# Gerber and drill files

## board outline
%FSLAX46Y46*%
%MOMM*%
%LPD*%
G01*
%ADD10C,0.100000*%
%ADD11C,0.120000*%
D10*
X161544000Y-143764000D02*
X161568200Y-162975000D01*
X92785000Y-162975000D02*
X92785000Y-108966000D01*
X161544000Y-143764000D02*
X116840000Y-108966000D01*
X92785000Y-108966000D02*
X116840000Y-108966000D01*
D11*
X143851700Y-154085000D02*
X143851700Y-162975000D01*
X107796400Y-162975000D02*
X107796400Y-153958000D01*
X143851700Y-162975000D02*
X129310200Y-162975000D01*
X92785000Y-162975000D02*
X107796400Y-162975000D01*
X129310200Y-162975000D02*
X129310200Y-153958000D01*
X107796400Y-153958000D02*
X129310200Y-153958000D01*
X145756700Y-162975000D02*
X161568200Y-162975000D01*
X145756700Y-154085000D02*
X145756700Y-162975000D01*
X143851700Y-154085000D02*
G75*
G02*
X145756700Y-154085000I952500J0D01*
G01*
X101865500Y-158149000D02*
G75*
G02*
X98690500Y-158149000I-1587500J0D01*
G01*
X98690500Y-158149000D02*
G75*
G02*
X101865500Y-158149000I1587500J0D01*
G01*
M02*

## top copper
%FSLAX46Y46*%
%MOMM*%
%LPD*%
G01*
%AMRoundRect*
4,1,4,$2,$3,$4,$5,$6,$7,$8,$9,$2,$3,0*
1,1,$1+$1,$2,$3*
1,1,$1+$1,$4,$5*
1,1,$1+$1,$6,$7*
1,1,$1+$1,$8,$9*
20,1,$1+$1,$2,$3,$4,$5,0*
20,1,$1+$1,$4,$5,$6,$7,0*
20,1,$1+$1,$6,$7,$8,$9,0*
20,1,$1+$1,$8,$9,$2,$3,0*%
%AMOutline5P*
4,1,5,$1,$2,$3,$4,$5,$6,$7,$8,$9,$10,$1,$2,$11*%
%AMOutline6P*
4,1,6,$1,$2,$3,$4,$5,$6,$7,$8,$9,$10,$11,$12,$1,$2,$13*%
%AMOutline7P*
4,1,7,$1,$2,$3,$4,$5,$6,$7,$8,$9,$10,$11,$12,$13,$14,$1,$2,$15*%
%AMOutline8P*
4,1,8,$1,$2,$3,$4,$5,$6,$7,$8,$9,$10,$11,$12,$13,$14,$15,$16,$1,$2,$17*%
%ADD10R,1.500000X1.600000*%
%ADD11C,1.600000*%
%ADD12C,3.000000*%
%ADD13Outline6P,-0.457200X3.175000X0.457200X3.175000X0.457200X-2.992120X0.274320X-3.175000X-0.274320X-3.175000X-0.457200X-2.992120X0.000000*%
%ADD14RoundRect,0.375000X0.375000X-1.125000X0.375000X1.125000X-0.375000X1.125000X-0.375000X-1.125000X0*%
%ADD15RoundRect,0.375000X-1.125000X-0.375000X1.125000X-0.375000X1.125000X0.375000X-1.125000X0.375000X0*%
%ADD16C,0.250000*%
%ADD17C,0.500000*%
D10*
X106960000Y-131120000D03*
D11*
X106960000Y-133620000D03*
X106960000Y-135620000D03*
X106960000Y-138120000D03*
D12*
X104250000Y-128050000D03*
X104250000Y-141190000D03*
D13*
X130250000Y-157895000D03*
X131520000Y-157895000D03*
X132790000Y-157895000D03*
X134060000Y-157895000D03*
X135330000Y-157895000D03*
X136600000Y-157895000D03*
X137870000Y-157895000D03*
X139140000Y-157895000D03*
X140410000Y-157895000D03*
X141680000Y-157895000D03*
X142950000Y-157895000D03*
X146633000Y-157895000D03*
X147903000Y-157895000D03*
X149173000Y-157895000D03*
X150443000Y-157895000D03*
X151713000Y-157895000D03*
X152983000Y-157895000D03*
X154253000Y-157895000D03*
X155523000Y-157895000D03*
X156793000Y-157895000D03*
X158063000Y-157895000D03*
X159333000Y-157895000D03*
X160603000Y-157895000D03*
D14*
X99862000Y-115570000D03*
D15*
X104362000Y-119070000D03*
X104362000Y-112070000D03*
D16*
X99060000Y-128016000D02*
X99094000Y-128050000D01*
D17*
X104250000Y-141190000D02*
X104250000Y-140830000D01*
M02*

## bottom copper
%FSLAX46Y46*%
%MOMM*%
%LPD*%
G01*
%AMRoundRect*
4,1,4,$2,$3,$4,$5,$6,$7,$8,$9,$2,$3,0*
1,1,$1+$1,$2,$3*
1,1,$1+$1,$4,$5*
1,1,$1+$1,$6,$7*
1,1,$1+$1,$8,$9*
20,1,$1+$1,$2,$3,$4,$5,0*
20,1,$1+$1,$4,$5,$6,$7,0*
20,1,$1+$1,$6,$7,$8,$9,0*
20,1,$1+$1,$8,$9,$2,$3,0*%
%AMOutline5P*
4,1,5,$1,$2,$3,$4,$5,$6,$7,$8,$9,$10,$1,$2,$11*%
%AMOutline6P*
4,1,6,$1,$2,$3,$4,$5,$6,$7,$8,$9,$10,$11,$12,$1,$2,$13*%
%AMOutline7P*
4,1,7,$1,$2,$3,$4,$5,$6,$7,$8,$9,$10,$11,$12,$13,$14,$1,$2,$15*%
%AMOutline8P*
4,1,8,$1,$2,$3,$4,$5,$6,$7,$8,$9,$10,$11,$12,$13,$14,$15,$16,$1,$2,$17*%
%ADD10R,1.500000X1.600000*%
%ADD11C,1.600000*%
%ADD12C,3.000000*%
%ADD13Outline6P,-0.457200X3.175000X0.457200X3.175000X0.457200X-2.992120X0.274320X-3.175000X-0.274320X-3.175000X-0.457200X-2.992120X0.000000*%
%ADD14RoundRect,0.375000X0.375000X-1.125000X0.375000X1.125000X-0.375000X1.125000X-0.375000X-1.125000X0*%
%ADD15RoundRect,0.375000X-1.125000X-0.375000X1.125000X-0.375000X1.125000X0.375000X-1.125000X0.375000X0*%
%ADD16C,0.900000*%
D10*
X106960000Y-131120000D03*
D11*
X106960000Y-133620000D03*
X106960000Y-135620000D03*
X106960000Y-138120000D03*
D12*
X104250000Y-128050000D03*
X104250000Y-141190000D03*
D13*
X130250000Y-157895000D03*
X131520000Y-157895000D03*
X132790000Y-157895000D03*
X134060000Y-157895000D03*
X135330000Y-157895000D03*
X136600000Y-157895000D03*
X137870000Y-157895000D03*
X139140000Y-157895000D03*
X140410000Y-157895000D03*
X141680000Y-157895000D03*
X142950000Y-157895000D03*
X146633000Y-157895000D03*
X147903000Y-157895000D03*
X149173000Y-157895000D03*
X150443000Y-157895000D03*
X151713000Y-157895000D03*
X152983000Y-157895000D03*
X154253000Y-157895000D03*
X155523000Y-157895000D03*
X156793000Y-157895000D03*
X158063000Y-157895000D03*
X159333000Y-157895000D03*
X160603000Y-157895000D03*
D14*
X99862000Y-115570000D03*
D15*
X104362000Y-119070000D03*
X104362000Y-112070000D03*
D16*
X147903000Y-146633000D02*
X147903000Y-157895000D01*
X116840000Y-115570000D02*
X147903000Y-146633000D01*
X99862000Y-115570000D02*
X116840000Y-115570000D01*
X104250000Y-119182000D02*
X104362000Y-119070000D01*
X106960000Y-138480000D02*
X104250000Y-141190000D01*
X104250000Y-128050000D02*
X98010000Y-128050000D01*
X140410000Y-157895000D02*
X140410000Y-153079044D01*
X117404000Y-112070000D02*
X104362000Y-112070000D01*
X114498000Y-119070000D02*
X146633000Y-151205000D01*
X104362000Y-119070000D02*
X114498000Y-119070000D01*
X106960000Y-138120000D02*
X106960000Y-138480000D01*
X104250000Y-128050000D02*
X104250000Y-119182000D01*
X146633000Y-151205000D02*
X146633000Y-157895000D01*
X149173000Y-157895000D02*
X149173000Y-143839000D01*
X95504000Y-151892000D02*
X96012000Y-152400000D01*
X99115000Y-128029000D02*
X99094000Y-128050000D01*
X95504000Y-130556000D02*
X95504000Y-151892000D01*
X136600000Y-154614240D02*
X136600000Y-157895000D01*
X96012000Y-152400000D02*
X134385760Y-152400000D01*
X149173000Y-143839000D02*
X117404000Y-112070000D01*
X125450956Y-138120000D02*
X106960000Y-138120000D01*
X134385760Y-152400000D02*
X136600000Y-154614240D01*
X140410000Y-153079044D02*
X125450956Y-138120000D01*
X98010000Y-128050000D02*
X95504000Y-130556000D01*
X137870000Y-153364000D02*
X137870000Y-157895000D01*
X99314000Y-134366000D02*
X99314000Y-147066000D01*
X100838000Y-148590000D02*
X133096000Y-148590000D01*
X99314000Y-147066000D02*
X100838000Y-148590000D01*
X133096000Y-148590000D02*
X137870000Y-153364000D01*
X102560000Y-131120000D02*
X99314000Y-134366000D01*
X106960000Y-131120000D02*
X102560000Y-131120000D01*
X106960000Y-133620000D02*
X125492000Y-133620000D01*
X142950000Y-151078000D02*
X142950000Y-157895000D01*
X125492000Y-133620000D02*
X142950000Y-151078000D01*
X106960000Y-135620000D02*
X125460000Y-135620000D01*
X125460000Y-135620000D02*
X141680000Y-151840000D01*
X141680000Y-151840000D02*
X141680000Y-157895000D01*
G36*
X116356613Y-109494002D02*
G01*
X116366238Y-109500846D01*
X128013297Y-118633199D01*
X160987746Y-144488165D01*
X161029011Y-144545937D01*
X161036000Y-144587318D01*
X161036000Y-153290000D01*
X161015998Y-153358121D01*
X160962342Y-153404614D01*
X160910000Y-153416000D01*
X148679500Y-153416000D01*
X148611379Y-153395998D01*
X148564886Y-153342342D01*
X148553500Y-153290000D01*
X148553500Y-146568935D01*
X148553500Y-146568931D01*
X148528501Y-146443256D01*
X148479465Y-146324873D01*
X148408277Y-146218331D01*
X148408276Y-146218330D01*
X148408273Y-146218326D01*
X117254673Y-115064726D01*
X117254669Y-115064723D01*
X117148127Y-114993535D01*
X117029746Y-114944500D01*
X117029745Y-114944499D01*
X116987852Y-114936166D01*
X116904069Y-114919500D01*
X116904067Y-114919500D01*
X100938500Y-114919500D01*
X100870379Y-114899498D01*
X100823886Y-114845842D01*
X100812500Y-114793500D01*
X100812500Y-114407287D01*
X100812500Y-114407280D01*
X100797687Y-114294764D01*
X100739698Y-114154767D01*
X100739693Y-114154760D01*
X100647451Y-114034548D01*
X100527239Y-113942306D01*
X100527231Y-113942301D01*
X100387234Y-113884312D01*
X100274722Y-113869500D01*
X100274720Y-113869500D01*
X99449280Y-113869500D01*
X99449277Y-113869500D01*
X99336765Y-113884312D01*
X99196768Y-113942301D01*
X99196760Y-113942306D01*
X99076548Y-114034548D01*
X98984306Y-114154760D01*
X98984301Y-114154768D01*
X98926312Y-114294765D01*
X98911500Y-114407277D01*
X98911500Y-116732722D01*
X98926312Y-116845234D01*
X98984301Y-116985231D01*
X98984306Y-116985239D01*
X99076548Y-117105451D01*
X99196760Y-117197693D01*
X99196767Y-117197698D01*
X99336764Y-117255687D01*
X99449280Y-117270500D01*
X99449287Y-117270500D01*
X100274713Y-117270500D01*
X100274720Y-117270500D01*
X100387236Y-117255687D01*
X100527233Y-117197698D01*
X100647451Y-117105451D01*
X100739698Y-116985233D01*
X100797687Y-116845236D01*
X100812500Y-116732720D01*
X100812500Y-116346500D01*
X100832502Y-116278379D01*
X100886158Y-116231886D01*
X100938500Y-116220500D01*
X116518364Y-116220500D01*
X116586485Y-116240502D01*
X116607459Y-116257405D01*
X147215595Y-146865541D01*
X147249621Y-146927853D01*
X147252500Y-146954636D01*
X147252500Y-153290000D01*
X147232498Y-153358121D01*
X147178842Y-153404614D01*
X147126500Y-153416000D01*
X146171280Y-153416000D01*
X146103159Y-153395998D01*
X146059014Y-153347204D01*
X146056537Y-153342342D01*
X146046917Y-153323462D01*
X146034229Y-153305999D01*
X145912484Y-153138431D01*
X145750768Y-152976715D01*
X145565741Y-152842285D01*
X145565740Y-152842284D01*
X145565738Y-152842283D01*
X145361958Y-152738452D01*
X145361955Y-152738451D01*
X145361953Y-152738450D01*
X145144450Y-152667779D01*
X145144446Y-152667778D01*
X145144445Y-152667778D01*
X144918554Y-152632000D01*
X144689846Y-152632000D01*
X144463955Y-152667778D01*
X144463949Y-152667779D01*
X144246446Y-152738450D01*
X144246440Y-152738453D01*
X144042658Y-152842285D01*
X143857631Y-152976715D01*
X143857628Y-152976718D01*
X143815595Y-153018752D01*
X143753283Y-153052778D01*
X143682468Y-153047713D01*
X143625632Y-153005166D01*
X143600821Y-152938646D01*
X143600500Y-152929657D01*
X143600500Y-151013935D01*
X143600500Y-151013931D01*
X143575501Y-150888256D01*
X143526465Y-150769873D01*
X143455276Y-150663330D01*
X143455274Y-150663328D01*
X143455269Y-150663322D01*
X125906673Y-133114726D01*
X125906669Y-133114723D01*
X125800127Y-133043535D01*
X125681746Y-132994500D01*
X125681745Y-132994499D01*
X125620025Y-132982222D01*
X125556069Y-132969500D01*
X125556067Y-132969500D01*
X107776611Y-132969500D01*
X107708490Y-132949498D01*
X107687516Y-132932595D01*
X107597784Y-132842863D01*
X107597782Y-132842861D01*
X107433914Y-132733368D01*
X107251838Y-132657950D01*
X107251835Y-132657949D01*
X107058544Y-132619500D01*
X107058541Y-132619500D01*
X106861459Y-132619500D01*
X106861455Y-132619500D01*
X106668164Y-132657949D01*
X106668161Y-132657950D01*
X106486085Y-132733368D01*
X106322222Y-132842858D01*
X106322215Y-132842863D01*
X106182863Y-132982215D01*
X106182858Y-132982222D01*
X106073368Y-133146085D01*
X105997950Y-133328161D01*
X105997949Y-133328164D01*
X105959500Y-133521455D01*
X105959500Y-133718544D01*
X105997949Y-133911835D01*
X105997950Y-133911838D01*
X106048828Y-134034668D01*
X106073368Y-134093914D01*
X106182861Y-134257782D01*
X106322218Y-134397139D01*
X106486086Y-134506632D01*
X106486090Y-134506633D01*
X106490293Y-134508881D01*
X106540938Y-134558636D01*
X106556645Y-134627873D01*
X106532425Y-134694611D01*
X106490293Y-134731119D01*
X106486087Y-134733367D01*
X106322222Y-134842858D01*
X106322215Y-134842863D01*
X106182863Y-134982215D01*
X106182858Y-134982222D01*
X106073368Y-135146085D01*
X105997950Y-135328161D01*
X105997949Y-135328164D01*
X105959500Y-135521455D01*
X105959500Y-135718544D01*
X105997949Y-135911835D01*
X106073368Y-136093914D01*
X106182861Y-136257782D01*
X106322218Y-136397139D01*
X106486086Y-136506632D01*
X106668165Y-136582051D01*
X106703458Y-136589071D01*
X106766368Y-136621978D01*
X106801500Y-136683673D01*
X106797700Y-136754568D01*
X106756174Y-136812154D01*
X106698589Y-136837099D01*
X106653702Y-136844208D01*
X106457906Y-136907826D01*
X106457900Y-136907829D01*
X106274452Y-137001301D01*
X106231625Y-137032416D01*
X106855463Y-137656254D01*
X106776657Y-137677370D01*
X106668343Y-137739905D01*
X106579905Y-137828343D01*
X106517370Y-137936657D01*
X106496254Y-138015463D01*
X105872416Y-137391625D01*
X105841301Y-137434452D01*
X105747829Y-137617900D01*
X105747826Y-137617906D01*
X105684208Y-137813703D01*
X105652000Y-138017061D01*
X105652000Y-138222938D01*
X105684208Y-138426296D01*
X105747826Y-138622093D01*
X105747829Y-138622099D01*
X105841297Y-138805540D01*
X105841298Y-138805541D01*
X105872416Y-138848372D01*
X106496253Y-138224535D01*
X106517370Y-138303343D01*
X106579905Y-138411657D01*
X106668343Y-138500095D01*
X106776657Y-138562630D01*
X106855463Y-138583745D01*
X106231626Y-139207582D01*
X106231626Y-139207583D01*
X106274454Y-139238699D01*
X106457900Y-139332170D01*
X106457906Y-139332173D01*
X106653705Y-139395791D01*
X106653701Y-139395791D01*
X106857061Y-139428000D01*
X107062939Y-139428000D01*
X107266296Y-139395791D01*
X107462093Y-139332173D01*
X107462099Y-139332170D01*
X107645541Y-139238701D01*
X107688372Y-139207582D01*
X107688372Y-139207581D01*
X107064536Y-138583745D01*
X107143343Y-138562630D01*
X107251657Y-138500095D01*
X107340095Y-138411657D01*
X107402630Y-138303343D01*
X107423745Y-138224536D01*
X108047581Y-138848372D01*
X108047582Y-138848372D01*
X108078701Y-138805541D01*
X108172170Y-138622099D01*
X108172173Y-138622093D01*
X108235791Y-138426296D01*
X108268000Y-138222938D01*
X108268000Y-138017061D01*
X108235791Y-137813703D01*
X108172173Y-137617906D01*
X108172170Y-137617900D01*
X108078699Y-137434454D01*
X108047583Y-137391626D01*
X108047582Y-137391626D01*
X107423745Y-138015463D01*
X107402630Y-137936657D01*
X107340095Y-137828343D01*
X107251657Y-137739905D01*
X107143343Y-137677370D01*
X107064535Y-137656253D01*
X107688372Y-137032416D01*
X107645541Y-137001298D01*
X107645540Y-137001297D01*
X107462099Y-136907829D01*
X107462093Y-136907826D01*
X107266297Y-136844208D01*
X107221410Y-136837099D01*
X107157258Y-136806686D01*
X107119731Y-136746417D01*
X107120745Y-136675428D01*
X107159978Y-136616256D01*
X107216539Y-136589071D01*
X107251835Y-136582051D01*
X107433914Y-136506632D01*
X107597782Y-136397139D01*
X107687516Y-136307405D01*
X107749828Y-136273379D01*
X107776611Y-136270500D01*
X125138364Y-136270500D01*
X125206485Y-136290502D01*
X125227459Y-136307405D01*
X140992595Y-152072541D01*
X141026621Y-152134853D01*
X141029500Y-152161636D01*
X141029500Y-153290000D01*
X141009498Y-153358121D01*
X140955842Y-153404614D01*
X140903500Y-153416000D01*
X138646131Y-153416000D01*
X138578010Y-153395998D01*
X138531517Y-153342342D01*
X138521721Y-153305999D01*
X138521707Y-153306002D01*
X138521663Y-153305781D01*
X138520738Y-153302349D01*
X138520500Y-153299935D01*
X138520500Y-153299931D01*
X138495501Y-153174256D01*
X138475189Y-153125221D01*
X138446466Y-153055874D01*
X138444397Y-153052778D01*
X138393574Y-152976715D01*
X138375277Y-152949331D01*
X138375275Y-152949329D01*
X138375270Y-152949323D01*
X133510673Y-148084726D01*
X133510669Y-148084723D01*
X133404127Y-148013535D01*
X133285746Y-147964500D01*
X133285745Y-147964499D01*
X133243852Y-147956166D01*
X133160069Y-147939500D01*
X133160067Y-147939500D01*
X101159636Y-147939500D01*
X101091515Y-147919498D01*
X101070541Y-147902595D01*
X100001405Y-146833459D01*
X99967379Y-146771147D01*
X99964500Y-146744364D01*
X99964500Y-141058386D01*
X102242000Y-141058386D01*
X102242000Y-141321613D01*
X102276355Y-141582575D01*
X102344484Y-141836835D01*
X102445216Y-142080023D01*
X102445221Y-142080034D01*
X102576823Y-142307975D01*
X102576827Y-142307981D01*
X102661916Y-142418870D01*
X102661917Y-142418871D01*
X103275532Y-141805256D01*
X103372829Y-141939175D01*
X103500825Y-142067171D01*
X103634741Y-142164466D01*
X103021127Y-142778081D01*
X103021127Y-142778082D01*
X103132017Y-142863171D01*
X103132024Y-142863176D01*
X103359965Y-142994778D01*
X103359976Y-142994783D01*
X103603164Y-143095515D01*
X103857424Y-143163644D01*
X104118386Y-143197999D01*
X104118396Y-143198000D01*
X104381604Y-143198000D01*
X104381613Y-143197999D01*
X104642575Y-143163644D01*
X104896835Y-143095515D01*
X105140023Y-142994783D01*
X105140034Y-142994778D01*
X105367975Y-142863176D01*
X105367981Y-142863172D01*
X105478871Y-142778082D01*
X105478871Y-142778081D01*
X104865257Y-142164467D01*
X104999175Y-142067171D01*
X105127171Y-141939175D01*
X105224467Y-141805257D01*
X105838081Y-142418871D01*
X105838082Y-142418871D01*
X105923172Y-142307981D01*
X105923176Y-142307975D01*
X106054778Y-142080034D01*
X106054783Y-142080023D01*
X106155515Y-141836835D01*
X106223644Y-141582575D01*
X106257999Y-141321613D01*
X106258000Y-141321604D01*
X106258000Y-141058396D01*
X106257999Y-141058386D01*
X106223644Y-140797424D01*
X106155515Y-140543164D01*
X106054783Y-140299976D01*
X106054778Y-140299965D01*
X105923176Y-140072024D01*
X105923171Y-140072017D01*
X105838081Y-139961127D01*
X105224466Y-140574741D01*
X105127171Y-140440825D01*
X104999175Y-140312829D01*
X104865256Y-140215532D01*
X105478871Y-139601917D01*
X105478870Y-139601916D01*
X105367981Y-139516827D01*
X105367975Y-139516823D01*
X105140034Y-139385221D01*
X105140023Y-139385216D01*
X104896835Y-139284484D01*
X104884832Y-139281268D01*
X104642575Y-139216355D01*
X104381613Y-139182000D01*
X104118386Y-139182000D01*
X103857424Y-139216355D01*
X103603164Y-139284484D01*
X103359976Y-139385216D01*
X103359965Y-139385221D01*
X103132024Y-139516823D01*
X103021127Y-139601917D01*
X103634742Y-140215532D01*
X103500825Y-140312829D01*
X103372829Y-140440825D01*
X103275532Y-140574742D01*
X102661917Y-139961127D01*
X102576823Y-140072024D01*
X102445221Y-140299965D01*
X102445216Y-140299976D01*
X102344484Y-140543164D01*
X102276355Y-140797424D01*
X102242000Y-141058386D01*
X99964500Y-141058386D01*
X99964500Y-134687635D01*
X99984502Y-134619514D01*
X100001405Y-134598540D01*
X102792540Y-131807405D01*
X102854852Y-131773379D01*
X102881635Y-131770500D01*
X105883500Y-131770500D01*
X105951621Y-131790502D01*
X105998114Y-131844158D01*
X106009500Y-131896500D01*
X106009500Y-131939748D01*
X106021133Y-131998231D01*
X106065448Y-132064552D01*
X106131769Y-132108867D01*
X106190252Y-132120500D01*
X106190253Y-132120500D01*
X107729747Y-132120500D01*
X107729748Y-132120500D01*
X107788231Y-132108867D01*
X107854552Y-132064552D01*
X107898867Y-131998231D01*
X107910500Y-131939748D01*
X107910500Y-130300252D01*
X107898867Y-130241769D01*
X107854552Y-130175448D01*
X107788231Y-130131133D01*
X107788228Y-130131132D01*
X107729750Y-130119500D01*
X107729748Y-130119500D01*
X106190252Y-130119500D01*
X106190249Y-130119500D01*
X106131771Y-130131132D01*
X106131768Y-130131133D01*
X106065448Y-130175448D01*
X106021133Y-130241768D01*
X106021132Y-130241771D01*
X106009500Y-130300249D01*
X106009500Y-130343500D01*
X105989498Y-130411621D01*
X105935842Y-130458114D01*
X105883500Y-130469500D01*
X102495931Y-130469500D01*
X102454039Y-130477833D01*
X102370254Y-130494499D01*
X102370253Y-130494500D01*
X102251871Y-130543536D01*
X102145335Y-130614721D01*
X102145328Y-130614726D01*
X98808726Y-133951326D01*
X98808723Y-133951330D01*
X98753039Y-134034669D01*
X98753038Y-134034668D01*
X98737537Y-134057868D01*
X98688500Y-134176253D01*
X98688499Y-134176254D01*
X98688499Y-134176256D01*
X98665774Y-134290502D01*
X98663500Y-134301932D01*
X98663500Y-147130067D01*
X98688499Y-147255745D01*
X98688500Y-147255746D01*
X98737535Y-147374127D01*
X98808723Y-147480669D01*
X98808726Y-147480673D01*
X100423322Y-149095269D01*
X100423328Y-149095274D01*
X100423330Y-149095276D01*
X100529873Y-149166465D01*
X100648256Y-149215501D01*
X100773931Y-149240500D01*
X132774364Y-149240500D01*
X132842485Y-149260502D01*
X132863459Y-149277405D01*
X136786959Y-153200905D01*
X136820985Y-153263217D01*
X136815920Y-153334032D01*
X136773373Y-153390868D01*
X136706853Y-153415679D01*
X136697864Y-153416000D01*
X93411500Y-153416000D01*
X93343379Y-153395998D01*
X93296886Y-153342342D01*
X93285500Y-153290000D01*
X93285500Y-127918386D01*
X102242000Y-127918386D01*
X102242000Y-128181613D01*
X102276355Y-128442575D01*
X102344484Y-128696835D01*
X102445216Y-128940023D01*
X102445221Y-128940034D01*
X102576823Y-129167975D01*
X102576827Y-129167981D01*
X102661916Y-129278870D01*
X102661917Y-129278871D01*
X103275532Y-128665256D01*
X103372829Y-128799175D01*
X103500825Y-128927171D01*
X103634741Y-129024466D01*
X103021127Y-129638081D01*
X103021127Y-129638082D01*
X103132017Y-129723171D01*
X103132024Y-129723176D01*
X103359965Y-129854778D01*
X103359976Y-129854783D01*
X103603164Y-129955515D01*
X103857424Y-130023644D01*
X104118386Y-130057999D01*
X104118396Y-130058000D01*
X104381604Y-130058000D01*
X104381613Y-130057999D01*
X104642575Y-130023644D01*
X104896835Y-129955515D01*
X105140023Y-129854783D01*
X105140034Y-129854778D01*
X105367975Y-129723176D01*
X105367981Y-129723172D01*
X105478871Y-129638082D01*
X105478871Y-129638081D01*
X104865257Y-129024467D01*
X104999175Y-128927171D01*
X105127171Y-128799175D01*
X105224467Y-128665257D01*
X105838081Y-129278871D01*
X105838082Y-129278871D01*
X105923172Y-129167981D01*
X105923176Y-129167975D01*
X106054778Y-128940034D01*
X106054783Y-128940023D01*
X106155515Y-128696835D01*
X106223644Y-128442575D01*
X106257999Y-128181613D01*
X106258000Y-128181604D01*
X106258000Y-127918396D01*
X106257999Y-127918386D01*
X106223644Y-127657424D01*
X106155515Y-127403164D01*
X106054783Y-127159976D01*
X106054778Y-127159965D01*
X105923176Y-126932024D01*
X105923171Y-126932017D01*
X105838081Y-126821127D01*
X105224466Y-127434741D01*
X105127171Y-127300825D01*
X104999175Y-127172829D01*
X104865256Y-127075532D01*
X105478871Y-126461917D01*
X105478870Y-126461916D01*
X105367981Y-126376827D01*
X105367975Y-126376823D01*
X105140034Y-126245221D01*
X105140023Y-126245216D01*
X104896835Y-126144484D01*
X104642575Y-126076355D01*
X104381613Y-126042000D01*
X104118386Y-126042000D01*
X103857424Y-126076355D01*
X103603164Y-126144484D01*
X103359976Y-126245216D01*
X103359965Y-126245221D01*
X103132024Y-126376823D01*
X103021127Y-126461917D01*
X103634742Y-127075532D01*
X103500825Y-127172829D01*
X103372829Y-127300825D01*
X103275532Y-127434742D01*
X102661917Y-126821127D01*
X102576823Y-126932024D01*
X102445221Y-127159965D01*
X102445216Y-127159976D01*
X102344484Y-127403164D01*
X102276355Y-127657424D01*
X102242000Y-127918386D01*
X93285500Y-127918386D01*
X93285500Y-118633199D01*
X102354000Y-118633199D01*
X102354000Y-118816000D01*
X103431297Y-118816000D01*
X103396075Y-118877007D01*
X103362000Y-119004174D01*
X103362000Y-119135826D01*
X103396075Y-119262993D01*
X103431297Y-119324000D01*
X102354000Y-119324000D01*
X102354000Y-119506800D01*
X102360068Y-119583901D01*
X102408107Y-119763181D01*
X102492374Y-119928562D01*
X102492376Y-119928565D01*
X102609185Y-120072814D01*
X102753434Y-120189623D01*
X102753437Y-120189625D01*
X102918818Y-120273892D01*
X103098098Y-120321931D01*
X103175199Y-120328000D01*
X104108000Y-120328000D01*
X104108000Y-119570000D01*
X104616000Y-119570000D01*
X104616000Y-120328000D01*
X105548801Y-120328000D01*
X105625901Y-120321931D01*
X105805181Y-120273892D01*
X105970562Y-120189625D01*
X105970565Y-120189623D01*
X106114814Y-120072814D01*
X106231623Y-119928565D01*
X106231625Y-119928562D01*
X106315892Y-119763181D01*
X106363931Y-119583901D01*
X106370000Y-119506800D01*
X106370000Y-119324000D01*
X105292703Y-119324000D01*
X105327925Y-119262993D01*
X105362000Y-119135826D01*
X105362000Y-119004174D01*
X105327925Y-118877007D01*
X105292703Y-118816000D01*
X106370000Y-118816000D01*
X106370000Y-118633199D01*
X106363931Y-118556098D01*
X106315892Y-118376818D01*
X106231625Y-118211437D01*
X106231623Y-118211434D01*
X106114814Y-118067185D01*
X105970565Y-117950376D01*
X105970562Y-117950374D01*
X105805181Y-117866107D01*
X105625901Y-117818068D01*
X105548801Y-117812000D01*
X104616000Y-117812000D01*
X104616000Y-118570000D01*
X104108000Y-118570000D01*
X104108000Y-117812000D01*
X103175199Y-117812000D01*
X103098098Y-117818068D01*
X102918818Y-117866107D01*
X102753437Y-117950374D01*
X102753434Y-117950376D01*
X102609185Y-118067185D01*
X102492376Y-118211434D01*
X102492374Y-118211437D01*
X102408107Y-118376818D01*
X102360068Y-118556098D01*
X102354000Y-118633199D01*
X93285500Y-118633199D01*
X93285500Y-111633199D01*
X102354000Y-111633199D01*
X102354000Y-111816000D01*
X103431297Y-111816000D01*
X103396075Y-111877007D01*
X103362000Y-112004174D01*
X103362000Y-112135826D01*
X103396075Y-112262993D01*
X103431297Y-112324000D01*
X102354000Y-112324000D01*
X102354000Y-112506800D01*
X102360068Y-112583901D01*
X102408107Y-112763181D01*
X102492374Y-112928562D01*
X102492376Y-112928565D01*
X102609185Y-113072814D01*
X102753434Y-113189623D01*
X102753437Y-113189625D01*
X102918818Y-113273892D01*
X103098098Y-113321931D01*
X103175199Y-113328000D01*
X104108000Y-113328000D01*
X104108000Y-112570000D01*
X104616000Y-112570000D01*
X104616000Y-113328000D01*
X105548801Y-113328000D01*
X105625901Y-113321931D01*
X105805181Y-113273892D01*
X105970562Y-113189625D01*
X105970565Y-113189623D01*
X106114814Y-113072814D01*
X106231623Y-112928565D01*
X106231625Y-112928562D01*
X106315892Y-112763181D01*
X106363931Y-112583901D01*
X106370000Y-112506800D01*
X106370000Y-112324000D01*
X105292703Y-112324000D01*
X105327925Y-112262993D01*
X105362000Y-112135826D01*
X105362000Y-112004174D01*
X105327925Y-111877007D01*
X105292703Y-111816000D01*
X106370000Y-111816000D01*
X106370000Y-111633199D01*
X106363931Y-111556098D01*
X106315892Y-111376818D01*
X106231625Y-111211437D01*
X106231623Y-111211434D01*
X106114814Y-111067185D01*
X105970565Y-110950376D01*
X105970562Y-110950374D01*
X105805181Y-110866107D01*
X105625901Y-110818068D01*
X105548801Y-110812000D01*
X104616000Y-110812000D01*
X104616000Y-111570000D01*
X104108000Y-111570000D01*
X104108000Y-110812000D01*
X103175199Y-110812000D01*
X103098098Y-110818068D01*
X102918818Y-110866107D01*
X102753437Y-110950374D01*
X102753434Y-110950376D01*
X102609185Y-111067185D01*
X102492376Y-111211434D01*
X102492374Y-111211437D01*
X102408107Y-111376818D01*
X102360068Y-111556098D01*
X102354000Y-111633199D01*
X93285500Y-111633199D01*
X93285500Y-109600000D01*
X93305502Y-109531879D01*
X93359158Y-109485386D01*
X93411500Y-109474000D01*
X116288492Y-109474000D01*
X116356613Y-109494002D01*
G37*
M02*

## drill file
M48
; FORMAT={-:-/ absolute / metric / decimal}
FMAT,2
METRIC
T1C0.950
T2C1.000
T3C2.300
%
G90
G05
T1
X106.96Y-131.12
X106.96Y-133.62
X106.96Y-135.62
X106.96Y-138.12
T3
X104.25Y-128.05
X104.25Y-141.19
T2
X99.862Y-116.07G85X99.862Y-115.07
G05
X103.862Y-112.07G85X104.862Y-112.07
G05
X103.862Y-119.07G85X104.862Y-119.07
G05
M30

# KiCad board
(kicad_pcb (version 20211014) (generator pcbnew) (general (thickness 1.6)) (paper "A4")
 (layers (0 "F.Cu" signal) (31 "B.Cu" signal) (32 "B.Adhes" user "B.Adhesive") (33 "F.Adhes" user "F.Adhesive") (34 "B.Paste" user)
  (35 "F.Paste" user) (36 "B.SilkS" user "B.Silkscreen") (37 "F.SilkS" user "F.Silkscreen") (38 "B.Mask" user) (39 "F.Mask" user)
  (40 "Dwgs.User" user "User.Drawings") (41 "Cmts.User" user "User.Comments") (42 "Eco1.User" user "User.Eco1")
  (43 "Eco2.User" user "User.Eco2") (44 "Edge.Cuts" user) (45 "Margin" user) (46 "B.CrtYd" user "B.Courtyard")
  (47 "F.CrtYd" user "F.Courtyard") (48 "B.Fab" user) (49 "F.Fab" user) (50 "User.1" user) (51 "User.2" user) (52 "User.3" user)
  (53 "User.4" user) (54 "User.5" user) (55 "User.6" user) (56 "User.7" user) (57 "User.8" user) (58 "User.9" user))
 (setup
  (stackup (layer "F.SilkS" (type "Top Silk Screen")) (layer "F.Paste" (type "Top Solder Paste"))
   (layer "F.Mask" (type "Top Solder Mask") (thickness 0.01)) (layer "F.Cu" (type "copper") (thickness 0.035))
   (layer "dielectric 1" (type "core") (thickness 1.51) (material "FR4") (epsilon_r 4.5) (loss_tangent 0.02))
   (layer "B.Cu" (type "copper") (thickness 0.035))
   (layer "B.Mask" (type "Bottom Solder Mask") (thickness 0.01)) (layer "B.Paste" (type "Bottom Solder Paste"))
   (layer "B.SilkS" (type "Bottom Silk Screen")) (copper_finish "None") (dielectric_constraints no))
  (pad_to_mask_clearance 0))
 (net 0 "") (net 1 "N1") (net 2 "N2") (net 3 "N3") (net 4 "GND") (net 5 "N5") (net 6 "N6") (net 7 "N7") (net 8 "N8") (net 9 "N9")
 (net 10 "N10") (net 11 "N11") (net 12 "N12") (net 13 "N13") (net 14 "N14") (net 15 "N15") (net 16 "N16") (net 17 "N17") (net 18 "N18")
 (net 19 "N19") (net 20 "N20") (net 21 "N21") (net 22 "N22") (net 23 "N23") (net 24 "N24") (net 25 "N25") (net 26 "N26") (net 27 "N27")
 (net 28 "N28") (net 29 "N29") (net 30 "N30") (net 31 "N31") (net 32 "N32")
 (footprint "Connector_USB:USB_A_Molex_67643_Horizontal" (layer "F.Cu") (at 106.96 131.12 -90)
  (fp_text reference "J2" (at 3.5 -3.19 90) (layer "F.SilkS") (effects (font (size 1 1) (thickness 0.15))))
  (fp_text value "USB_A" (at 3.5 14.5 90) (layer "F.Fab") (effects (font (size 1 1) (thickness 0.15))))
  (pad "1" thru_hole rect (at 0 0 270) (size 1.6 1.5) (drill 0.95) (layers *.Cu *.Mask) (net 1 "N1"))
  (pad "2" thru_hole circle (at 2.5 0 270) (size 1.6 1.6) (drill 0.95) (layers *.Cu *.Mask) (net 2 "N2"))
  (pad "3" thru_hole circle (at 4.5 0 270) (size 1.6 1.6) (drill 0.95) (layers *.Cu *.Mask) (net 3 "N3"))
  (pad "4" thru_hole circle (at 7 0 270) (size 1.6 1.6) (drill 0.95) (layers *.Cu *.Mask) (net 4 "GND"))
  (pad "5" thru_hole circle (at -3.07 2.71 270) (size 3 3) (drill 2.3) (layers *.Cu *.Mask) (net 4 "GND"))
  (pad "5" thru_hole circle (at 10.07 2.71 270) (size 3 3) (drill 2.3) (layers *.Cu *.Mask) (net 4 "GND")))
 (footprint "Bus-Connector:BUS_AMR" (layer "F.Cu") (at 92.785 162.975)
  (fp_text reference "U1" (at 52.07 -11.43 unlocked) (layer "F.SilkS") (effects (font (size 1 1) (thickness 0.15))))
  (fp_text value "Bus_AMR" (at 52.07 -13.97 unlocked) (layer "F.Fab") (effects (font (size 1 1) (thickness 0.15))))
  (fp_line (start 51.0667 -8.89) (end 51.0667 0) (layer "Edge.Cuts") (width 0.12))
  (fp_line (start 15.0114 0) (end 15.0114 -9.017) (layer "Edge.Cuts") (width 0.12))
  (fp_line (start 51.0667 0) (end 36.5252 0) (layer "Edge.Cuts") (width 0.12))
  (fp_line (start 0 0) (end 15.0114 0) (layer "Edge.Cuts") (width 0.12))
  (fp_line (start 36.5252 0) (end 36.5252 -9.017) (layer "Edge.Cuts") (width 0.12))
  (fp_line (start 15.0114 -9.017) (end 36.5252 -9.017) (layer "Edge.Cuts") (width 0.12))
  (fp_line (start 52.9717 0) (end 68.7832 0) (layer "Edge.Cuts") (width 0.12))
  (fp_line (start 52.9717 -8.89) (end 52.9717 0) (layer "Edge.Cuts") (width 0.12))
  (fp_arc (start 51.0667 -8.89) (mid 52.0192 -9.8425) (end 52.9717 -8.89) (layer "Edge.Cuts") (width 0.12))
  (fp_circle (center 7.493 -4.826) (end 9.0805 -4.826) (layer "Edge.Cuts") (width 0.12) (fill none))
  (pad "A1" connect roundrect (at 37.465 -5.08) (size 0.9144 6.35) (layers "B.Cu" "B.Mask") (roundrect_rratio 0) (chamfer_ratio 0.2)
   (chamfer bottom_left bottom_right) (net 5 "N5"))
  (pad "A2" connect roundrect (at 38.735 -5.08) (size 0.9144 6.35) (layers "B.Cu" "B.Mask") (roundrect_rratio 0) (chamfer_ratio 0.2)
   (chamfer bottom_left bottom_right) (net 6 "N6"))
  (pad "A3" connect roundrect (at 40.005 -5.08) (size 0.9144 6.35) (layers "B.Cu" "B.Mask") (roundrect_rratio 0) (chamfer_ratio 0.2)
   (chamfer bottom_left bottom_right) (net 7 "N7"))
  (pad "A4" connect roundrect (at 41.275 -5.08) (size 0.9144 6.35) (layers "B.Cu" "B.Mask") (roundrect_rratio 0) (chamfer_ratio 0.2)
   (chamfer bottom_left bottom_right) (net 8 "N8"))
  (pad "A5" connect roundrect (at 42.545 -5.08) (size 0.9144 6.35) (layers "B.Cu" "B.Mask") (roundrect_rratio 0) (chamfer_ratio 0.2)
   (chamfer bottom_left bottom_right) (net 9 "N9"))
  (pad "A6" connect roundrect (at 43.815 -5.08) (size 0.9144 6.35) (layers "B.Cu" "B.Mask") (roundrect_rratio 0) (chamfer_ratio 0.2)
   (chamfer bottom_left bottom_right) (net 4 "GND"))
  (pad "A7" connect roundrect (at 45.085 -5.08) (size 0.9144 6.35) (layers "B.Cu" "B.Mask") (roundrect_rratio 0) (chamfer_ratio 0.2)
   (chamfer bottom_left bottom_right) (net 1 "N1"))
  (pad "A8" connect roundrect (at 46.355 -5.08) (size 0.9144 6.35) (layers "B.Cu" "B.Mask") (roundrect_rratio 0) (chamfer_ratio 0.2)
   (chamfer bottom_left bottom_right) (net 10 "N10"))
  (pad "A9" connect roundrect (at 47.625 -5.08) (size 0.9144 6.35) (layers "B.Cu" "B.Mask") (roundrect_rratio 0) (chamfer_ratio 0.2)
   (chamfer bottom_left bottom_right) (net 4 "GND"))
  (pad "A10" connect roundrect (at 48.895 -5.08) (size 0.9144 6.35) (layers "B.Cu" "B.Mask") (roundrect_rratio 0) (chamfer_ratio 0.2)
   (chamfer bottom_left bottom_right) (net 3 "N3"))
  (pad "A11" connect roundrect (at 50.165 -5.08) (size 0.9144 6.35) (layers "B.Cu" "B.Mask") (roundrect_rratio 0) (chamfer_ratio 0.2)
   (chamfer bottom_left bottom_right) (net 2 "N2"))
  (pad "A12" connect roundrect (at 53.848 -5.08) (size 0.9144 6.35) (layers "B.Cu" "B.Mask") (roundrect_rratio 0) (chamfer_ratio 0.2)
   (chamfer bottom_left bottom_right) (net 4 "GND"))
  (pad "A13" connect roundrect (at 55.118 -5.08) (size 0.9144 6.35) (layers "B.Cu" "B.Mask") (roundrect_rratio 0) (chamfer_ratio 0.2)
   (chamfer bottom_left bottom_right) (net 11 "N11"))
  (pad "A14" connect roundrect (at 56.388 -5.08) (size 0.9144 6.35) (layers "B.Cu" "B.Mask") (roundrect_rratio 0) (chamfer_ratio 0.2)
   (chamfer bottom_left bottom_right) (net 4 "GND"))
  (pad "A15" connect roundrect (at 57.658 -5.08) (size 0.9144 6.35) (layers "B.Cu" "B.Mask") (roundrect_rratio 0) (chamfer_ratio 0.2)
   (chamfer bottom_left bottom_right) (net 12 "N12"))
  (pad "A16" connect roundrect (at 58.928 -5.08) (size 0.9144 6.35) (layers "B.Cu" "B.Mask") (roundrect_rratio 0) (chamfer_ratio 0.2)
   (chamfer bottom_left bottom_right) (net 4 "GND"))
  (pad "A17" connect roundrect (at 60.198 -5.08) (size 0.9144 6.35) (layers "B.Cu" "B.Mask") (roundrect_rratio 0) (chamfer_ratio 0.2)
   (chamfer bottom_left bottom_right) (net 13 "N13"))
  (pad "A18" connect roundrect (at 61.468 -5.08) (size 0.9144 6.35) (layers "B.Cu" "B.Mask") (roundrect_rratio 0) (chamfer_ratio 0.2)
   (chamfer bottom_left bottom_right) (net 4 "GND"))
  (pad "A19" connect roundrect (at 62.738 -5.08) (size 0.9144 6.35) (layers "B.Cu" "B.Mask") (roundrect_rratio 0) (chamfer_ratio 0.2)
   (chamfer bottom_left bottom_right) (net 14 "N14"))
  (pad "A20" connect roundrect (at 64.008 -5.08) (size 0.9144 6.35) (layers "B.Cu" "B.Mask") (roundrect_rratio 0) (chamfer_ratio 0.2)
   (chamfer bottom_left bottom_right) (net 4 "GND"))
  (pad "A21" connect roundrect (at 65.278 -5.08) (size 0.9144 6.35) (layers "B.Cu" "B.Mask") (roundrect_rratio 0) (chamfer_ratio 0.2)
   (chamfer bottom_left bottom_right) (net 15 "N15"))
  (pad "A22" connect roundrect (at 66.548 -5.08) (size 0.9144 6.35) (layers "B.Cu" "B.Mask") (roundrect_rratio 0) (chamfer_ratio 0.2)
   (chamfer bottom_left bottom_right) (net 4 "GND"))
  (pad "A23" connect roundrect (at 67.818 -5.08) (size 0.9144 6.35) (layers "B.Cu" "B.Mask") (roundrect_rratio 0) (chamfer_ratio 0.2)
   (chamfer bottom_left bottom_right) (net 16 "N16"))
  (pad "B1" connect roundrect (at 37.465 -5.08) (size 0.9144 6.35) (layers "F.Cu" "F.Mask") (roundrect_rratio 0) (chamfer_ratio 0.2)
   (chamfer bottom_left bottom_right) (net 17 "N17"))
  (pad "B2" connect roundrect (at 38.735 -5.08) (size 0.9144 6.35) (layers "F.Cu" "F.Mask") (roundrect_rratio 0) (chamfer_ratio 0.2)
   (chamfer bottom_left bottom_right) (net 4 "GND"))
  (pad "B3" connect roundrect (at 40.005 -5.08) (size 0.9144 6.35) (layers "F.Cu" "F.Mask") (roundrect_rratio 0) (chamfer_ratio 0.2)
   (chamfer bottom_left bottom_right) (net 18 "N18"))
  (pad "B4" connect roundrect (at 41.275 -5.08) (size 0.9144 6.35) (layers "F.Cu" "F.Mask") (roundrect_rratio 0) (chamfer_ratio 0.2)
   (chamfer bottom_left bottom_right) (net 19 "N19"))
  (pad "B5" connect roundrect (at 42.545 -5.08) (size 0.9144 6.35) (layers "F.Cu" "F.Mask") (roundrect_rratio 0) (chamfer_ratio 0.2)
   (chamfer bottom_left bottom_right) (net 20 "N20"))
  (pad "B6" connect roundrect (at 43.815 -5.08) (size 0.9144 6.35) (layers "F.Cu" "F.Mask") (roundrect_rratio 0) (chamfer_ratio 0.2)
   (chamfer bottom_left bottom_right) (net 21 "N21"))
  (pad "B7" connect roundrect (at 45.085 -5.08) (size 0.9144 6.35) (layers "F.Cu" "F.Mask") (roundrect_rratio 0) (chamfer_ratio 0.2)
   (chamfer bottom_left bottom_right) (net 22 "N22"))
  (pad "B8" connect roundrect (at 46.355 -5.08) (size 0.9144 6.35) (layers "F.Cu" "F.Mask") (roundrect_rratio 0) (chamfer_ratio 0.2)
   (chamfer bottom_left bottom_right) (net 4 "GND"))
  (pad "B9" connect roundrect (at 47.625 -5.08) (size 0.9144 6.35) (layers "F.Cu" "F.Mask") (roundrect_rratio 0) (chamfer_ratio 0.2)
   (chamfer bottom_left bottom_right) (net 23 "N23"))
  (pad "B10" connect roundrect (at 48.895 -5.08) (size 0.9144 6.35) (layers "F.Cu" "F.Mask") (roundrect_rratio 0) (chamfer_ratio 0.2)
   (chamfer bottom_left bottom_right) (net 4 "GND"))
  (pad "B11" connect roundrect (at 50.165 -5.08) (size 0.9144 6.35) (layers "F.Cu" "F.Mask") (roundrect_rratio 0) (chamfer_ratio 0.2)
   (chamfer bottom_left bottom_right) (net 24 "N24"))
  (pad "B12" connect roundrect (at 53.848 -5.08) (size 0.9144 6.35) (layers "F.Cu" "F.Mask") (roundrect_rratio 0) (chamfer_ratio 0.2)
   (chamfer bottom_left bottom_right) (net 4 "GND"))
  (pad "B13" connect roundrect (at 55.118 -5.08) (size 0.9144 6.35) (layers "F.Cu" "F.Mask") (roundrect_rratio 0) (chamfer_ratio 0.2)
   (chamfer bottom_left bottom_right) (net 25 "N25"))
  (pad "B14" connect roundrect (at 56.388 -5.08) (size 0.9144 6.35) (layers "F.Cu" "F.Mask") (roundrect_rratio 0) (chamfer_ratio 0.2)
   (chamfer bottom_left bottom_right) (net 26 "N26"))
  (pad "B15" connect roundrect (at 57.658 -5.08) (size 0.9144 6.35) (layers "F.Cu" "F.Mask") (roundrect_rratio 0) (chamfer_ratio 0.2)
   (chamfer bottom_left bottom_right) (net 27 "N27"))
  (pad "B16" connect roundrect (at 58.928 -5.08) (size 0.9144 6.35) (layers "F.Cu" "F.Mask") (roundrect_rratio 0) (chamfer_ratio 0.2)
   (chamfer bottom_left bottom_right) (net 4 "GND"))
  (pad "B17" connect roundrect (at 60.198 -5.08) (size 0.9144 6.35) (layers "F.Cu" "F.Mask") (roundrect_rratio 0) (chamfer_ratio 0.2)
   (chamfer bottom_left bottom_right) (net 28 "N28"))
  (pad "B18" connect roundrect (at 61.468 -5.08) (size 0.9144 6.35) (layers "F.Cu" "F.Mask") (roundrect_rratio 0) (chamfer_ratio 0.2)
   (chamfer bottom_left bottom_right) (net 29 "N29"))
  (pad "B19" connect roundrect (at 62.738 -5.08) (size 0.9144 6.35) (layers "F.Cu" "F.Mask") (roundrect_rratio 0) (chamfer_ratio 0.2)
   (chamfer bottom_left bottom_right) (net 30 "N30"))
  (pad "B20" connect roundrect (at 64.008 -5.08) (size 0.9144 6.35) (layers "F.Cu" "F.Mask") (roundrect_rratio 0) (chamfer_ratio 0.2)
   (chamfer bottom_left bottom_right) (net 4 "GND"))
  (pad "B21" connect roundrect (at 65.278 -5.08) (size 0.9144 6.35) (layers "F.Cu" "F.Mask") (roundrect_rratio 0) (chamfer_ratio 0.2)
   (chamfer bottom_left bottom_right) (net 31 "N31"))
  (pad "B22" connect roundrect (at 66.548 -5.08) (size 0.9144 6.35) (layers "F.Cu" "F.Mask") (roundrect_rratio 0) (chamfer_ratio 0.2)
   (chamfer bottom_left bottom_right) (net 4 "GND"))
  (pad "B23" connect roundrect (at 67.818 -5.08) (size 0.9144 6.35) (layers "F.Cu" "F.Mask") (roundrect_rratio 0) (chamfer_ratio 0.2)
   (chamfer bottom_left bottom_right) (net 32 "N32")))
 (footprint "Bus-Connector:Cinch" (layer "F.Cu") (at 102.362 115.57)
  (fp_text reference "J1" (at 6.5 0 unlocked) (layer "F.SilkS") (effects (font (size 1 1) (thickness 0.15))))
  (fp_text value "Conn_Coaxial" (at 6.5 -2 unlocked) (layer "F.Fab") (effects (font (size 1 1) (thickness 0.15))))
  (pad "1" thru_hole roundrect (at -2.5 0 90) (size 3 1.5) (drill oval 2 1) (layers *.Cu *.Mask) (roundrect_rratio 0.25) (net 11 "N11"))
  (pad "2" thru_hole roundrect (at 2 3.5) (size 3 1.5) (drill oval 2 1) (layers *.Cu *.Mask) (roundrect_rratio 0.25) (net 4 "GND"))
  (pad "2" thru_hole roundrect (at 2 -3.5) (size 3 1.5) (drill oval 2 1) (layers *.Cu *.Mask) (roundrect_rratio 0.25) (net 4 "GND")))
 (gr_line (start 161.544 143.764) (end 161.5682 162.975) (layer "Edge.Cuts") (width 0.1))
 (gr_line (start 92.785 162.975) (end 92.785 108.966) (layer "Edge.Cuts") (width 0.1))
 (gr_line (start 161.544 143.764) (end 116.84 108.966) (layer "Edge.Cuts") (width 0.1))
 (gr_line (start 92.785 108.966) (end 116.84 108.966) (layer "Edge.Cuts") (width 0.1))
 (segment (start 147.903 146.633) (end 147.903 157.895) (width 0.9) (layer "B.Cu") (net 11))
 (segment (start 116.84 115.57) (end 147.903 146.633) (width 0.9) (layer "B.Cu") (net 11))
 (segment (start 99.862 115.57) (end 116.84 115.57) (width 0.9) (layer "B.Cu") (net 11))
 (segment (start 99.06 128.016) (end 99.094 128.05) (width 0.25) (layer "F.Cu") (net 4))
 (segment (start 104.25 141.19) (end 104.25 140.83) (width 0.5) (layer "F.Cu") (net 4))
 (segment (start 104.25 119.182) (end 104.362 119.07) (width 0.9) (layer "B.Cu") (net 4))
 (segment (start 106.96 138.48) (end 104.25 141.19) (width 0.9) (layer "B.Cu") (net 4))
 (segment (start 104.25 128.05) (end 98.01 128.05) (width 0.9) (layer "B.Cu") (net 4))
 (segment (start 140.41 157.895) (end 140.41 153.079044) (width 0.9) (layer "B.Cu") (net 4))
 (segment (start 117.404 112.07) (end 104.362 112.07) (width 0.9) (layer "B.Cu") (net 4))
 (segment (start 114.498 119.07) (end 146.633 151.205) (width 0.9) (layer "B.Cu") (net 4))
 (segment (start 104.362 119.07) (end 114.498 119.07) (width 0.9) (layer "B.Cu") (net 4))
 (segment (start 106.96 138.12) (end 106.96 138.48) (width 0.9) (layer "B.Cu") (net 4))
 (segment (start 104.25 128.05) (end 104.25 119.182) (width 0.9) (layer "B.Cu") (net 4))
 (segment (start 146.633 151.205) (end 146.633 157.895) (width 0.9) (layer "B.Cu") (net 4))
 (segment (start 149.173 157.895) (end 149.173 143.839) (width 0.9) (layer "B.Cu") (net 4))
 (segment (start 95.504 151.892) (end 96.012 152.4) (width 0.9) (layer "B.Cu") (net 4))
 (segment (start 99.115 128.029) (end 99.094 128.05) (width 0.9) (layer "B.Cu") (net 4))
 (segment (start 95.504 130.556) (end 95.504 151.892) (width 0.9) (layer "B.Cu") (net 4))
 (segment (start 136.6 154.61424) (end 136.6 157.895) (width 0.9) (layer "B.Cu") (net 4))
 (segment (start 96.012 152.4) (end 134.38576 152.4) (width 0.9) (layer "B.Cu") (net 4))
 (segment (start 149.173 143.839) (end 117.404 112.07) (width 0.9) (layer "B.Cu") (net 4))
 (segment (start 125.450956 138.12) (end 106.96 138.12) (width 0.9) (layer "B.Cu") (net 4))
 (segment (start 134.38576 152.4) (end 136.6 154.61424) (width 0.9) (layer "B.Cu") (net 4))
 (segment (start 140.41 153.079044) (end 125.450956 138.12) (width 0.9) (layer "B.Cu") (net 4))
 (segment (start 98.01 128.05) (end 95.504 130.556) (width 0.9) (layer "B.Cu") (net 4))
 (segment (start 137.87 153.364) (end 137.87 157.895) (width 0.9) (layer "B.Cu") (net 1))
 (segment (start 99.314 134.366) (end 99.314 147.066) (width 0.9) (layer "B.Cu") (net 1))
 (segment (start 100.838 148.59) (end 133.096 148.59) (width 0.9) (layer "B.Cu") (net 1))
 (segment (start 99.314 147.066) (end 100.838 148.59) (width 0.9) (layer "B.Cu") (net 1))
 (segment (start 133.096 148.59) (end 137.87 153.364) (width 0.9) (layer "B.Cu") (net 1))
 (segment (start 102.56 131.12) (end 99.314 134.366) (width 0.9) (layer "B.Cu") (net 1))
 (segment (start 106.96 131.12) (end 102.56 131.12) (width 0.9) (layer "B.Cu") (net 1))
 (segment (start 106.96 133.62) (end 125.492 133.62) (width 0.9) (layer "B.Cu") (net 2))
 (segment (start 142.95 151.078) (end 142.95 157.895) (width 0.9) (layer "B.Cu") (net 2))
 (segment (start 125.492 133.62) (end 142.95 151.078) (width 0.9) (layer "B.Cu") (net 2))
 (segment (start 106.96 135.62) (end 125.46 135.62) (width 0.9) (layer "B.Cu") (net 3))
 (segment (start 125.46 135.62) (end 141.68 151.84) (width 0.9) (layer "B.Cu") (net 3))
 (segment (start 141.68 151.84) (end 141.68 157.895) (width 0.9) (layer "B.Cu") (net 3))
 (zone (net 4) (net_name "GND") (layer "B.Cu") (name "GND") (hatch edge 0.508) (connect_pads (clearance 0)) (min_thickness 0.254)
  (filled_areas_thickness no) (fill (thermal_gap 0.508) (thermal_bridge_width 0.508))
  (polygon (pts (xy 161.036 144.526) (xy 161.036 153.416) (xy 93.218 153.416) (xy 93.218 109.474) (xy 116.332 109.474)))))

